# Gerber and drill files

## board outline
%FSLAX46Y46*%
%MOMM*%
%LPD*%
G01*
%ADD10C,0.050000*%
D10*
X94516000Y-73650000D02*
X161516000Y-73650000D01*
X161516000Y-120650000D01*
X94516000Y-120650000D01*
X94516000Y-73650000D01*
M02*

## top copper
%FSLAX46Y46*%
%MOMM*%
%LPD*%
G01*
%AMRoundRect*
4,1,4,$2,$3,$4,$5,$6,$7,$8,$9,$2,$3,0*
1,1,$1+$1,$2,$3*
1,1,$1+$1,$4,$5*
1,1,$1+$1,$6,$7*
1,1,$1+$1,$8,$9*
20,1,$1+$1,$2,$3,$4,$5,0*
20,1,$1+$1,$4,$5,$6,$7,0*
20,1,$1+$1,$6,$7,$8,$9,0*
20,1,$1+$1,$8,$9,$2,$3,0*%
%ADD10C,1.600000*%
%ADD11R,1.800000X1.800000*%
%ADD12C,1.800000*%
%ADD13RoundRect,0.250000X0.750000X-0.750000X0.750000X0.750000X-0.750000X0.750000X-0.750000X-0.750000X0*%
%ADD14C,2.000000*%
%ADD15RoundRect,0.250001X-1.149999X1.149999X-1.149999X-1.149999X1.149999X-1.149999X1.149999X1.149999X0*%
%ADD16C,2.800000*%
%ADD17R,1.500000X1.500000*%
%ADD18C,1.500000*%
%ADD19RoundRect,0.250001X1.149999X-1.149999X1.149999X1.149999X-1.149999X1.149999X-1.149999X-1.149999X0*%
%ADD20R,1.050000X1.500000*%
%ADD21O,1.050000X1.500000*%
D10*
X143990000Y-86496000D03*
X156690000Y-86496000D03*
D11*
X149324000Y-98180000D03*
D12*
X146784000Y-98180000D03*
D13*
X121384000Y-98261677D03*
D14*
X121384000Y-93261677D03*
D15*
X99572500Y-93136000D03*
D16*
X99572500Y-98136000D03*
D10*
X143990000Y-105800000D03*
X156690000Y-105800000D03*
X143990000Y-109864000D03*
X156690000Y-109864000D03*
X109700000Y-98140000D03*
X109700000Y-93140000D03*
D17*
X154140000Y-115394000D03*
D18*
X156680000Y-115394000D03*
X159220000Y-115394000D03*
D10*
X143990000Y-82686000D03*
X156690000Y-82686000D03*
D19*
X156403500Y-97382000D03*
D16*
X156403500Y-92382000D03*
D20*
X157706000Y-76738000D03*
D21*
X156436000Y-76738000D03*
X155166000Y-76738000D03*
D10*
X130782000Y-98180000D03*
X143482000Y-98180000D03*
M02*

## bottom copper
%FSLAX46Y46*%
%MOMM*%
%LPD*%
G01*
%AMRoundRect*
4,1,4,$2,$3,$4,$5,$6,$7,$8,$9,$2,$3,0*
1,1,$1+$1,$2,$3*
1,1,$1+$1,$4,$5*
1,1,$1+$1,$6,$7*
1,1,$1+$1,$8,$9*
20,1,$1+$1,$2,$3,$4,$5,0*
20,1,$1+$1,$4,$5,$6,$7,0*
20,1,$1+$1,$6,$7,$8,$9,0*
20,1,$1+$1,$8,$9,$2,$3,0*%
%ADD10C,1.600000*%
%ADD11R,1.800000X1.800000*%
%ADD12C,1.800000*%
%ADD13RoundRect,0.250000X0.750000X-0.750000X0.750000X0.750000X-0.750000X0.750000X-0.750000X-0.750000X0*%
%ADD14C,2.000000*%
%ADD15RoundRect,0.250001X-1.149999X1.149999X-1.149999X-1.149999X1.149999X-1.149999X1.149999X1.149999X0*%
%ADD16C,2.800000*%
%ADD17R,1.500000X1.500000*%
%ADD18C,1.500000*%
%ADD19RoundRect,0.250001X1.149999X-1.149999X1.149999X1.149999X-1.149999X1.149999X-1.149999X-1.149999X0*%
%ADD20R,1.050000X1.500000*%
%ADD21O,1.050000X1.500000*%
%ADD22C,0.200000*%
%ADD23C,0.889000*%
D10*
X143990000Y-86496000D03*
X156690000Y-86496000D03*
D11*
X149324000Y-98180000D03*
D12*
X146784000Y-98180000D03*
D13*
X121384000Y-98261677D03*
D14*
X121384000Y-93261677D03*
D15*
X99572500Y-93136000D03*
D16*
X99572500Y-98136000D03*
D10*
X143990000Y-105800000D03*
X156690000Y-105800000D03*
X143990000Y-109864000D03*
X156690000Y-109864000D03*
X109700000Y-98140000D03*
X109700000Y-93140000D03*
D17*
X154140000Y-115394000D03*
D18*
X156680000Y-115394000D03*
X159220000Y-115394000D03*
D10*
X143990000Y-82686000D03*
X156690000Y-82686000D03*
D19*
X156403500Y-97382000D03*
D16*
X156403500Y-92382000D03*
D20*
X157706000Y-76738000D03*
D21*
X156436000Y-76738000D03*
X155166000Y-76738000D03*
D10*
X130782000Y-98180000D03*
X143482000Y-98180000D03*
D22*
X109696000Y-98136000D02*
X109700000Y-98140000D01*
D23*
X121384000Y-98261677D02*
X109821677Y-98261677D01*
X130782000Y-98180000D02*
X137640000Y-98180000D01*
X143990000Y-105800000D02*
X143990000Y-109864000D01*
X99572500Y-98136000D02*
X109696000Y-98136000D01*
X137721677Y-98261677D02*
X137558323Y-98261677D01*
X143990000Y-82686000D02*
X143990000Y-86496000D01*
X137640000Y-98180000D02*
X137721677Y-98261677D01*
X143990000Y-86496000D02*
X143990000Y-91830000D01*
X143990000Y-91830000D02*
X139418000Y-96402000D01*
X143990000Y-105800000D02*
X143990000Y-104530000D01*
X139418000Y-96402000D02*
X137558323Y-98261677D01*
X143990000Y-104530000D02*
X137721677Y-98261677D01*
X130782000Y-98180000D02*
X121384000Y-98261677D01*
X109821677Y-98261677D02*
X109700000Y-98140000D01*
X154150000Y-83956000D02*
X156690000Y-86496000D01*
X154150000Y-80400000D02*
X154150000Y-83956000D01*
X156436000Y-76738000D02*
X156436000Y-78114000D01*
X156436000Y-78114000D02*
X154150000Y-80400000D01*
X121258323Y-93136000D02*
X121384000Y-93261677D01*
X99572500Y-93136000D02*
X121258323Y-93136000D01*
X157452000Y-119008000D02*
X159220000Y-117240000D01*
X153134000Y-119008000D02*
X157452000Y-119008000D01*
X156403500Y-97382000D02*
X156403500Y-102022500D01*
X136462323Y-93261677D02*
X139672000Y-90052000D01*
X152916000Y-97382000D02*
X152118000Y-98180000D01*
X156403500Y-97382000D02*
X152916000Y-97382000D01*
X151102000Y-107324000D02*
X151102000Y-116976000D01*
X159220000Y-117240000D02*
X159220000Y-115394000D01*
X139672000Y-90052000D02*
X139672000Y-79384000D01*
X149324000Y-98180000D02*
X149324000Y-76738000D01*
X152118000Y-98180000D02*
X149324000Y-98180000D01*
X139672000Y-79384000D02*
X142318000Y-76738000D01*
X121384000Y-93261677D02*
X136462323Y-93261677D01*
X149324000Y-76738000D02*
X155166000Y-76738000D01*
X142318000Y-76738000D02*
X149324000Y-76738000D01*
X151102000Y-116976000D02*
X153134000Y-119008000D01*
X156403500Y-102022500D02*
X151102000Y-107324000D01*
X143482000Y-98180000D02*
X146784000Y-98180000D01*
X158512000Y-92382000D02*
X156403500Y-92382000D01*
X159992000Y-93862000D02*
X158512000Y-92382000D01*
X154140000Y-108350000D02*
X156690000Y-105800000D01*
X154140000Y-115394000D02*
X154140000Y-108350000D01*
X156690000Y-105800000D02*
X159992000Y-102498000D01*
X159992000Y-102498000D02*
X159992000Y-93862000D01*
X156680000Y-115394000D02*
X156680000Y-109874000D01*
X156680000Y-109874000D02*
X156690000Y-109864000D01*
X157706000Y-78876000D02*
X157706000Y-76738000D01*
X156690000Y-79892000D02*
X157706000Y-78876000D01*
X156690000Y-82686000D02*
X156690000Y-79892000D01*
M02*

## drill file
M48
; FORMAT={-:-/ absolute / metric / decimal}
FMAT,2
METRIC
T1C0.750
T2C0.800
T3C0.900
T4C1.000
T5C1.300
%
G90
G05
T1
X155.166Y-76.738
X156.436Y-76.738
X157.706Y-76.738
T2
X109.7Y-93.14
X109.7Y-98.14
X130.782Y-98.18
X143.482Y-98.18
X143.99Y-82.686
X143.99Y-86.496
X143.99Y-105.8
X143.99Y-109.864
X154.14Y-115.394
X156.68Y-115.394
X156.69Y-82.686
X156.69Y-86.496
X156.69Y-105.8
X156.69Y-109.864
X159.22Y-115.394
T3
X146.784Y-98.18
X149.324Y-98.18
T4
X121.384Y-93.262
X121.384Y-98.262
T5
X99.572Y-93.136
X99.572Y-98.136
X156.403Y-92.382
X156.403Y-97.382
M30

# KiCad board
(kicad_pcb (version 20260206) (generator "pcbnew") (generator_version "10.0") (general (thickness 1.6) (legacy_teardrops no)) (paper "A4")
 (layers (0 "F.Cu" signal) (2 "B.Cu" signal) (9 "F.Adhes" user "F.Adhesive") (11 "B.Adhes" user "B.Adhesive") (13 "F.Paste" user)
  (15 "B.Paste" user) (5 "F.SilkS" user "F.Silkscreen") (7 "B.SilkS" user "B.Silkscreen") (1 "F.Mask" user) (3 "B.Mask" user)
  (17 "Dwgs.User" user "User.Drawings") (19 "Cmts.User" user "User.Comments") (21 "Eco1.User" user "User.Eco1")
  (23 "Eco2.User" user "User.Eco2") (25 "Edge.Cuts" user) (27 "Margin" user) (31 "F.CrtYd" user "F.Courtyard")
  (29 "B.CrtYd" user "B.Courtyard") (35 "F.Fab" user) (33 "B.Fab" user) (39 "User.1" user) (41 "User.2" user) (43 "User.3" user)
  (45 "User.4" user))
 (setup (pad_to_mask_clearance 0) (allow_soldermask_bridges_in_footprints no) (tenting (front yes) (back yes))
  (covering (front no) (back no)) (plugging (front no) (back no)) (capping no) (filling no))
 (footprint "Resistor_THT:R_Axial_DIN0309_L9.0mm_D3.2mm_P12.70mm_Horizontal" (layer "F.Cu") (at 143.99 86.496)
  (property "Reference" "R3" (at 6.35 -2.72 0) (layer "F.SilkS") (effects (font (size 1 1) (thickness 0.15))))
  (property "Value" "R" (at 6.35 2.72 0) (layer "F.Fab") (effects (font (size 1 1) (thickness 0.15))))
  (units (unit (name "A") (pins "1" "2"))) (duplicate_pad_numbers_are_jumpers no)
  (pad "1" thru_hole circle (at 0 0) (size 1.6 1.6) (drill 0.8) (layers "*.Cu" "*.Mask") (remove_unused_layers no) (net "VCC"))
  (pad "2" thru_hole circle (at 12.7 0) (size 1.6 1.6) (drill 0.8) (layers "*.Cu" "*.Mask") (remove_unused_layers no) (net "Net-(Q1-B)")))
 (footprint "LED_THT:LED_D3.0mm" (layer "F.Cu") (at 149.324 98.18 180)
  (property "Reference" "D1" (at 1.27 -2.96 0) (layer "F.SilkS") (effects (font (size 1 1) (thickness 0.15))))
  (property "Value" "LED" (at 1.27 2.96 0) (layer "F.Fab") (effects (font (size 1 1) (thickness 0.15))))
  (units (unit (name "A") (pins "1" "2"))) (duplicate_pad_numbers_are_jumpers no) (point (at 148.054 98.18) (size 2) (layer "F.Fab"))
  (pad "1" thru_hole rect (at 0 0 180) (size 1.8 1.8) (drill 0.9) (layers "*.Cu" "*.Mask") (remove_unused_layers no) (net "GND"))
  (pad "2" thru_hole circle (at 2.54 0 180) (size 1.8 1.8) (drill 0.9) (layers "*.Cu" "*.Mask") (remove_unused_layers no) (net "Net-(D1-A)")))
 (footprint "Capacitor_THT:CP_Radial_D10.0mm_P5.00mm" (layer "F.Cu") (at 121.384 98.261677 90)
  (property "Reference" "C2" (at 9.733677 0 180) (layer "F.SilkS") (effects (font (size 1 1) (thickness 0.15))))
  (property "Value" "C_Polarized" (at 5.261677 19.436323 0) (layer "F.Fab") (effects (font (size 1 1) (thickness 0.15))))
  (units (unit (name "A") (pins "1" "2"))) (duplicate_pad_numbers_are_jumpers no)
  (pad "1" thru_hole roundrect (at 0 0 90) (size 2 2) (drill 1) (layers "*.Cu" "*.Mask") (remove_unused_layers no) (roundrect_rratio 0.125)
   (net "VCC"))
  (pad "2" thru_hole circle (at 5 0 90) (size 2 2) (drill 1) (layers "*.Cu" "*.Mask") (remove_unused_layers no) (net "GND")))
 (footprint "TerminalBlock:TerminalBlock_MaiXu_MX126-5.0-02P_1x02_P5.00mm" (layer "F.Cu") (at 99.5725 93.136 -90)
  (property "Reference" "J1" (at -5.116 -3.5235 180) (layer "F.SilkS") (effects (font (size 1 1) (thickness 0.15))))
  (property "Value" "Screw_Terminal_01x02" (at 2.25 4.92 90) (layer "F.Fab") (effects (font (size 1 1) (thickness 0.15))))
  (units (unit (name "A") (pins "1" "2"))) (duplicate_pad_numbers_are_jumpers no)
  (pad "1" thru_hole roundrect (at 0 0 270) (size 2.8 2.8) (drill 1.3) (layers "*.Cu" "*.Mask") (remove_unused_layers no)
   (roundrect_rratio 0.089286) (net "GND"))
  (pad "2" thru_hole circle (at 5 0 270) (size 2.8 2.8) (drill 1.3) (layers "*.Cu" "*.Mask") (remove_unused_layers no) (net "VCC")))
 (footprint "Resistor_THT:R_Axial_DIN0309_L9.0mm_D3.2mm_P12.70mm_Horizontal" (layer "F.Cu") (at 143.99 105.8)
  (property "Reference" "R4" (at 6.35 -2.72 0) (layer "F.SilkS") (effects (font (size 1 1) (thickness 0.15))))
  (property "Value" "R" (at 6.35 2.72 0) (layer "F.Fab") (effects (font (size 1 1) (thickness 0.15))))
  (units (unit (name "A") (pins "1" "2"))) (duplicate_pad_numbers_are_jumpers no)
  (pad "1" thru_hole circle (at 0 0) (size 1.6 1.6) (drill 0.8) (layers "*.Cu" "*.Mask") (remove_unused_layers no) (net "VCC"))
  (pad "2" thru_hole circle (at 12.7 0) (size 1.6 1.6) (drill 0.8) (layers "*.Cu" "*.Mask") (remove_unused_layers no) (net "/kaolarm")))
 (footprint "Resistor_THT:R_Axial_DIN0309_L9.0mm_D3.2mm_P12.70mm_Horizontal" (layer "F.Cu") (at 143.99 109.864)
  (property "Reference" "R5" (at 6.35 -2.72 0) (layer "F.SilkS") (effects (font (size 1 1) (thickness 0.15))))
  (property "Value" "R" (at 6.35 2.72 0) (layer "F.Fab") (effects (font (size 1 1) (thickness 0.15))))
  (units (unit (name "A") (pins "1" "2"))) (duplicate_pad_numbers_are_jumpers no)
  (pad "1" thru_hole circle (at 0 0) (size 1.6 1.6) (drill 0.8) (layers "*.Cu" "*.Mask") (remove_unused_layers no) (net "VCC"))
  (pad "2" thru_hole circle (at 12.7 0) (size 1.6 1.6) (drill 0.8) (layers "*.Cu" "*.Mask") (remove_unused_layers no) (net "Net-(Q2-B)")))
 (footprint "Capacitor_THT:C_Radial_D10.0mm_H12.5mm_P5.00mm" (layer "F.Cu") (at 109.7 98.14 90)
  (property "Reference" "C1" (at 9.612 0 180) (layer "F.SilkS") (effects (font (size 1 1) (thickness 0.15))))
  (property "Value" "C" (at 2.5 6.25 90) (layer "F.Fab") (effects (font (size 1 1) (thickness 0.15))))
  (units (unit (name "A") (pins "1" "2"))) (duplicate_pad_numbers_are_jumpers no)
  (pad "1" thru_hole circle (at 0 0 90) (size 1.6 1.6) (drill 0.8) (layers "*.Cu" "*.Mask") (remove_unused_layers no) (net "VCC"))
  (pad "2" thru_hole circle (at 5 0 90) (size 1.6 1.6) (drill 0.8) (layers "*.Cu" "*.Mask") (remove_unused_layers no) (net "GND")))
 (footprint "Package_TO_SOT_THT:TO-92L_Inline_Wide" (layer "F.Cu") (at 154.14 115.394)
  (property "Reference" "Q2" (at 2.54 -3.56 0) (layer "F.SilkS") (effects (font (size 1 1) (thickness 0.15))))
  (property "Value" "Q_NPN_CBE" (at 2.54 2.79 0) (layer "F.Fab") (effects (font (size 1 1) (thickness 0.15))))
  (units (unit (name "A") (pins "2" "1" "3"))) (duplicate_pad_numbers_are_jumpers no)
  (pad "1" thru_hole rect (at 0 0) (size 1.5 1.5) (drill 0.8) (layers "*.Cu" "*.Mask") (remove_unused_layers no) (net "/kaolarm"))
  (pad "2" thru_hole circle (at 2.54 0) (size 1.5 1.5) (drill 0.8) (layers "*.Cu" "*.Mask") (remove_unused_layers no) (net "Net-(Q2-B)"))
  (pad "3" thru_hole circle (at 5.08 0) (size 1.5 1.5) (drill 0.8) (layers "*.Cu" "*.Mask") (remove_unused_layers no) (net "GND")))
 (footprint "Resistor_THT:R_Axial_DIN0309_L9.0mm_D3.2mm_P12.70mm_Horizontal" (layer "F.Cu") (at 143.99 82.686)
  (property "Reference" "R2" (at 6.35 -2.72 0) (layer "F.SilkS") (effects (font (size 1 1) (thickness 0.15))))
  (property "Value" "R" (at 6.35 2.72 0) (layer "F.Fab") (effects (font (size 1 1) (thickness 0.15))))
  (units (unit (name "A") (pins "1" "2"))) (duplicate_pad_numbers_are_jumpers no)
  (pad "1" thru_hole circle (at 0 0) (size 1.6 1.6) (drill 0.8) (layers "*.Cu" "*.Mask") (remove_unused_layers no) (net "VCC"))
  (pad "2" thru_hole circle (at 12.7 0) (size 1.6 1.6) (drill 0.8) (layers "*.Cu" "*.Mask") (remove_unused_layers no) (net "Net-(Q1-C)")))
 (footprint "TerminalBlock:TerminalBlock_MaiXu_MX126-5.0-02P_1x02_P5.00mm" (layer "F.Cu") (at 156.4035 97.382 90)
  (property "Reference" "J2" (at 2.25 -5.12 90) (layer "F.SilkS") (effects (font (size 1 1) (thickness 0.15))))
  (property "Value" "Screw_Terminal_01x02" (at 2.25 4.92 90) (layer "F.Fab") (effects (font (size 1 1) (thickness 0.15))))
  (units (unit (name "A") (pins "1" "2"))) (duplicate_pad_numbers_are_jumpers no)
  (pad "1" thru_hole roundrect (at 0 0 90) (size 2.8 2.8) (drill 1.3) (layers "*.Cu" "*.Mask") (remove_unused_layers no)
   (roundrect_rratio 0.089286) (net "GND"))
  (pad "2" thru_hole circle (at 5 0 90) (size 2.8 2.8) (drill 1.3) (layers "*.Cu" "*.Mask") (remove_unused_layers no) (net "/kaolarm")))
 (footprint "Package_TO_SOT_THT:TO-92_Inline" (layer "F.Cu") (at 157.706 76.738 180)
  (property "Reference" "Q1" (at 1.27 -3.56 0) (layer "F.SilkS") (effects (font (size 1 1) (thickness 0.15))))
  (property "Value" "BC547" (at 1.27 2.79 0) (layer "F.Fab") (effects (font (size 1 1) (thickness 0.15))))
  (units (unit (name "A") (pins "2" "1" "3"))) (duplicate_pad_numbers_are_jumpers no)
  (pad "1" thru_hole rect (at 0 0 180) (size 1.05 1.5) (drill 0.75) (layers "*.Cu" "*.Mask") (remove_unused_layers no) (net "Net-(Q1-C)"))
  (pad "2" thru_hole oval (at 1.27 0 180) (size 1.05 1.5) (drill 0.75) (layers "*.Cu" "*.Mask") (remove_unused_layers no) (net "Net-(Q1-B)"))
  (pad "3" thru_hole oval (at 2.54 0 180) (size 1.05 1.5) (drill 0.75) (layers "*.Cu" "*.Mask") (remove_unused_layers no) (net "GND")))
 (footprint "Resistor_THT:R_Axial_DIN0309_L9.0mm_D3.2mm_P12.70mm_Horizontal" (layer "F.Cu") (at 130.782 98.18)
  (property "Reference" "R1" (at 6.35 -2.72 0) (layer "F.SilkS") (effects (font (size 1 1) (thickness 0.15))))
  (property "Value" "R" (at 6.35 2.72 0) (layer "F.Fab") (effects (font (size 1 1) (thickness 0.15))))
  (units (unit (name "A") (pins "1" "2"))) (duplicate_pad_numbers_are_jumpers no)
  (pad "1" thru_hole circle (at 0 0) (size 1.6 1.6) (drill 0.8) (layers "*.Cu" "*.Mask") (remove_unused_layers no) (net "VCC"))
  (pad "2" thru_hole circle (at 12.7 0) (size 1.6 1.6) (drill 0.8) (layers "*.Cu" "*.Mask") (remove_unused_layers no) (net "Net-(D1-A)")))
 (gr_rect (start 94.516 73.65) (end 161.516 120.65) (stroke (width 0.05) (type default)) (fill no) (layer "Edge.Cuts"))
 (segment (start 109.696 98.136) (end 109.7 98.14) (width 0.2) (layer "B.Cu") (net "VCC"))
 (segment (start 121.384 98.261677) (end 109.821677 98.261677) (width 0.889) (layer "B.Cu") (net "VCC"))
 (segment (start 130.782 98.18) (end 137.64 98.18) (width 0.889) (layer "B.Cu") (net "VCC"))
 (segment (start 143.99 105.8) (end 143.99 109.864) (width 0.889) (layer "B.Cu") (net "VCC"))
 (segment (start 99.5725 98.136) (end 109.696 98.136) (width 0.889) (layer "B.Cu") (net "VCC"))
 (segment (start 137.721677 98.261677) (end 137.558323 98.261677) (width 0.889) (layer "B.Cu") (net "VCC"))
 (segment (start 143.99 82.686) (end 143.99 86.496) (width 0.889) (layer "B.Cu") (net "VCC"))
 (segment (start 137.64 98.18) (end 137.721677 98.261677) (width 0.889) (layer "B.Cu") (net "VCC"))
 (segment (start 143.99 86.496) (end 143.99 91.83) (width 0.889) (layer "B.Cu") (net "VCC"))
 (segment (start 143.99 91.83) (end 139.418 96.402) (width 0.889) (layer "B.Cu") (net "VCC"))
 (segment (start 143.99 105.8) (end 143.99 104.53) (width 0.889) (layer "B.Cu") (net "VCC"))
 (segment (start 139.418 96.402) (end 137.558323 98.261677) (width 0.889) (layer "B.Cu") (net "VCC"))
 (segment (start 143.99 104.53) (end 137.721677 98.261677) (width 0.889) (layer "B.Cu") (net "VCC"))
 (segment (start 130.782 98.18) (end 121.384 98.261677) (width 0.889) (layer "B.Cu") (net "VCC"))
 (segment (start 109.821677 98.261677) (end 109.7 98.14) (width 0.889) (layer "B.Cu") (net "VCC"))
 (segment (start 154.15 83.956) (end 156.69 86.496) (width 0.889) (layer "B.Cu") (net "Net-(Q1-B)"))
 (segment (start 154.15 80.4) (end 154.15 83.956) (width 0.889) (layer "B.Cu") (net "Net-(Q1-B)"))
 (segment (start 156.436 76.738) (end 156.436 78.114) (width 0.889) (layer "B.Cu") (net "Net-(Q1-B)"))
 (segment (start 156.436 78.114) (end 154.15 80.4) (width 0.889) (layer "B.Cu") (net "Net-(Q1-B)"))
 (segment (start 121.258323 93.136) (end 121.384 93.261677) (width 0.889) (layer "B.Cu") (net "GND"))
 (segment (start 99.5725 93.136) (end 121.258323 93.136) (width 0.889) (layer "B.Cu") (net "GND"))
 (segment (start 157.452 119.008) (end 159.22 117.24) (width 0.889) (layer "B.Cu") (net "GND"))
 (segment (start 153.134 119.008) (end 157.452 119.008) (width 0.889) (layer "B.Cu") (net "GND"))
 (segment (start 156.4035 97.382) (end 156.4035 102.0225) (width 0.889) (layer "B.Cu") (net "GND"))
 (segment (start 136.462323 93.261677) (end 139.672 90.052) (width 0.889) (layer "B.Cu") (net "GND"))
 (segment (start 152.916 97.382) (end 152.118 98.18) (width 0.889) (layer "B.Cu") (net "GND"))
 (segment (start 156.4035 97.382) (end 152.916 97.382) (width 0.889) (layer "B.Cu") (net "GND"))
 (segment (start 151.102 107.324) (end 151.102 116.976) (width 0.889) (layer "B.Cu") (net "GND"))
 (segment (start 159.22 117.24) (end 159.22 115.394) (width 0.889) (layer "B.Cu") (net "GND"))
 (segment (start 139.672 90.052) (end 139.672 79.384) (width 0.889) (layer "B.Cu") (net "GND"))
 (segment (start 149.324 98.18) (end 149.324 76.738) (width 0.889) (layer "B.Cu") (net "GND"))
 (segment (start 152.118 98.18) (end 149.324 98.18) (width 0.889) (layer "B.Cu") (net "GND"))
 (segment (start 139.672 79.384) (end 142.318 76.738) (width 0.889) (layer "B.Cu") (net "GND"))
 (segment (start 121.384 93.261677) (end 136.462323 93.261677) (width 0.889) (layer "B.Cu") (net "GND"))
 (segment (start 149.324 76.738) (end 155.166 76.738) (width 0.889) (layer "B.Cu") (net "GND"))
 (segment (start 142.318 76.738) (end 149.324 76.738) (width 0.889) (layer "B.Cu") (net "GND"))
 (segment (start 151.102 116.976) (end 153.134 119.008) (width 0.889) (layer "B.Cu") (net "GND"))
 (segment (start 156.4035 102.0225) (end 151.102 107.324) (width 0.889) (layer "B.Cu") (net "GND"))
 (segment (start 143.482 98.18) (end 146.784 98.18) (width 0.889) (layer "B.Cu") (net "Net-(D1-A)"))
 (segment (start 158.512 92.382) (end 156.4035 92.382) (width 0.889) (layer "B.Cu") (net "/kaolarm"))
 (segment (start 159.992 93.862) (end 158.512 92.382) (width 0.889) (layer "B.Cu") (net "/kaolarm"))
 (segment (start 154.14 108.35) (end 156.69 105.8) (width 0.889) (layer "B.Cu") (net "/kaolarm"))
 (segment (start 154.14 115.394) (end 154.14 108.35) (width 0.889) (layer "B.Cu") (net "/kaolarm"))
 (segment (start 156.69 105.8) (end 159.992 102.498) (width 0.889) (layer "B.Cu") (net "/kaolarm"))
 (segment (start 159.992 102.498) (end 159.992 93.862) (width 0.889) (layer "B.Cu") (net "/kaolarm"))
 (segment (start 156.68 115.394) (end 156.68 109.874) (width 0.889) (layer "B.Cu") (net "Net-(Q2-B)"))
 (segment (start 156.68 109.874) (end 156.69 109.864) (width 0.889) (layer "B.Cu") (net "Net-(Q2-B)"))
 (segment (start 157.706 78.876) (end 157.706 76.738) (width 0.889) (layer "B.Cu") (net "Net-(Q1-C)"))
 (segment (start 156.69 79.892) (end 157.706 78.876) (width 0.889) (layer "B.Cu") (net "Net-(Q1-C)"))
 (segment (start 156.69 82.686) (end 156.69 79.892) (width 0.889) (layer "B.Cu") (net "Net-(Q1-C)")))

